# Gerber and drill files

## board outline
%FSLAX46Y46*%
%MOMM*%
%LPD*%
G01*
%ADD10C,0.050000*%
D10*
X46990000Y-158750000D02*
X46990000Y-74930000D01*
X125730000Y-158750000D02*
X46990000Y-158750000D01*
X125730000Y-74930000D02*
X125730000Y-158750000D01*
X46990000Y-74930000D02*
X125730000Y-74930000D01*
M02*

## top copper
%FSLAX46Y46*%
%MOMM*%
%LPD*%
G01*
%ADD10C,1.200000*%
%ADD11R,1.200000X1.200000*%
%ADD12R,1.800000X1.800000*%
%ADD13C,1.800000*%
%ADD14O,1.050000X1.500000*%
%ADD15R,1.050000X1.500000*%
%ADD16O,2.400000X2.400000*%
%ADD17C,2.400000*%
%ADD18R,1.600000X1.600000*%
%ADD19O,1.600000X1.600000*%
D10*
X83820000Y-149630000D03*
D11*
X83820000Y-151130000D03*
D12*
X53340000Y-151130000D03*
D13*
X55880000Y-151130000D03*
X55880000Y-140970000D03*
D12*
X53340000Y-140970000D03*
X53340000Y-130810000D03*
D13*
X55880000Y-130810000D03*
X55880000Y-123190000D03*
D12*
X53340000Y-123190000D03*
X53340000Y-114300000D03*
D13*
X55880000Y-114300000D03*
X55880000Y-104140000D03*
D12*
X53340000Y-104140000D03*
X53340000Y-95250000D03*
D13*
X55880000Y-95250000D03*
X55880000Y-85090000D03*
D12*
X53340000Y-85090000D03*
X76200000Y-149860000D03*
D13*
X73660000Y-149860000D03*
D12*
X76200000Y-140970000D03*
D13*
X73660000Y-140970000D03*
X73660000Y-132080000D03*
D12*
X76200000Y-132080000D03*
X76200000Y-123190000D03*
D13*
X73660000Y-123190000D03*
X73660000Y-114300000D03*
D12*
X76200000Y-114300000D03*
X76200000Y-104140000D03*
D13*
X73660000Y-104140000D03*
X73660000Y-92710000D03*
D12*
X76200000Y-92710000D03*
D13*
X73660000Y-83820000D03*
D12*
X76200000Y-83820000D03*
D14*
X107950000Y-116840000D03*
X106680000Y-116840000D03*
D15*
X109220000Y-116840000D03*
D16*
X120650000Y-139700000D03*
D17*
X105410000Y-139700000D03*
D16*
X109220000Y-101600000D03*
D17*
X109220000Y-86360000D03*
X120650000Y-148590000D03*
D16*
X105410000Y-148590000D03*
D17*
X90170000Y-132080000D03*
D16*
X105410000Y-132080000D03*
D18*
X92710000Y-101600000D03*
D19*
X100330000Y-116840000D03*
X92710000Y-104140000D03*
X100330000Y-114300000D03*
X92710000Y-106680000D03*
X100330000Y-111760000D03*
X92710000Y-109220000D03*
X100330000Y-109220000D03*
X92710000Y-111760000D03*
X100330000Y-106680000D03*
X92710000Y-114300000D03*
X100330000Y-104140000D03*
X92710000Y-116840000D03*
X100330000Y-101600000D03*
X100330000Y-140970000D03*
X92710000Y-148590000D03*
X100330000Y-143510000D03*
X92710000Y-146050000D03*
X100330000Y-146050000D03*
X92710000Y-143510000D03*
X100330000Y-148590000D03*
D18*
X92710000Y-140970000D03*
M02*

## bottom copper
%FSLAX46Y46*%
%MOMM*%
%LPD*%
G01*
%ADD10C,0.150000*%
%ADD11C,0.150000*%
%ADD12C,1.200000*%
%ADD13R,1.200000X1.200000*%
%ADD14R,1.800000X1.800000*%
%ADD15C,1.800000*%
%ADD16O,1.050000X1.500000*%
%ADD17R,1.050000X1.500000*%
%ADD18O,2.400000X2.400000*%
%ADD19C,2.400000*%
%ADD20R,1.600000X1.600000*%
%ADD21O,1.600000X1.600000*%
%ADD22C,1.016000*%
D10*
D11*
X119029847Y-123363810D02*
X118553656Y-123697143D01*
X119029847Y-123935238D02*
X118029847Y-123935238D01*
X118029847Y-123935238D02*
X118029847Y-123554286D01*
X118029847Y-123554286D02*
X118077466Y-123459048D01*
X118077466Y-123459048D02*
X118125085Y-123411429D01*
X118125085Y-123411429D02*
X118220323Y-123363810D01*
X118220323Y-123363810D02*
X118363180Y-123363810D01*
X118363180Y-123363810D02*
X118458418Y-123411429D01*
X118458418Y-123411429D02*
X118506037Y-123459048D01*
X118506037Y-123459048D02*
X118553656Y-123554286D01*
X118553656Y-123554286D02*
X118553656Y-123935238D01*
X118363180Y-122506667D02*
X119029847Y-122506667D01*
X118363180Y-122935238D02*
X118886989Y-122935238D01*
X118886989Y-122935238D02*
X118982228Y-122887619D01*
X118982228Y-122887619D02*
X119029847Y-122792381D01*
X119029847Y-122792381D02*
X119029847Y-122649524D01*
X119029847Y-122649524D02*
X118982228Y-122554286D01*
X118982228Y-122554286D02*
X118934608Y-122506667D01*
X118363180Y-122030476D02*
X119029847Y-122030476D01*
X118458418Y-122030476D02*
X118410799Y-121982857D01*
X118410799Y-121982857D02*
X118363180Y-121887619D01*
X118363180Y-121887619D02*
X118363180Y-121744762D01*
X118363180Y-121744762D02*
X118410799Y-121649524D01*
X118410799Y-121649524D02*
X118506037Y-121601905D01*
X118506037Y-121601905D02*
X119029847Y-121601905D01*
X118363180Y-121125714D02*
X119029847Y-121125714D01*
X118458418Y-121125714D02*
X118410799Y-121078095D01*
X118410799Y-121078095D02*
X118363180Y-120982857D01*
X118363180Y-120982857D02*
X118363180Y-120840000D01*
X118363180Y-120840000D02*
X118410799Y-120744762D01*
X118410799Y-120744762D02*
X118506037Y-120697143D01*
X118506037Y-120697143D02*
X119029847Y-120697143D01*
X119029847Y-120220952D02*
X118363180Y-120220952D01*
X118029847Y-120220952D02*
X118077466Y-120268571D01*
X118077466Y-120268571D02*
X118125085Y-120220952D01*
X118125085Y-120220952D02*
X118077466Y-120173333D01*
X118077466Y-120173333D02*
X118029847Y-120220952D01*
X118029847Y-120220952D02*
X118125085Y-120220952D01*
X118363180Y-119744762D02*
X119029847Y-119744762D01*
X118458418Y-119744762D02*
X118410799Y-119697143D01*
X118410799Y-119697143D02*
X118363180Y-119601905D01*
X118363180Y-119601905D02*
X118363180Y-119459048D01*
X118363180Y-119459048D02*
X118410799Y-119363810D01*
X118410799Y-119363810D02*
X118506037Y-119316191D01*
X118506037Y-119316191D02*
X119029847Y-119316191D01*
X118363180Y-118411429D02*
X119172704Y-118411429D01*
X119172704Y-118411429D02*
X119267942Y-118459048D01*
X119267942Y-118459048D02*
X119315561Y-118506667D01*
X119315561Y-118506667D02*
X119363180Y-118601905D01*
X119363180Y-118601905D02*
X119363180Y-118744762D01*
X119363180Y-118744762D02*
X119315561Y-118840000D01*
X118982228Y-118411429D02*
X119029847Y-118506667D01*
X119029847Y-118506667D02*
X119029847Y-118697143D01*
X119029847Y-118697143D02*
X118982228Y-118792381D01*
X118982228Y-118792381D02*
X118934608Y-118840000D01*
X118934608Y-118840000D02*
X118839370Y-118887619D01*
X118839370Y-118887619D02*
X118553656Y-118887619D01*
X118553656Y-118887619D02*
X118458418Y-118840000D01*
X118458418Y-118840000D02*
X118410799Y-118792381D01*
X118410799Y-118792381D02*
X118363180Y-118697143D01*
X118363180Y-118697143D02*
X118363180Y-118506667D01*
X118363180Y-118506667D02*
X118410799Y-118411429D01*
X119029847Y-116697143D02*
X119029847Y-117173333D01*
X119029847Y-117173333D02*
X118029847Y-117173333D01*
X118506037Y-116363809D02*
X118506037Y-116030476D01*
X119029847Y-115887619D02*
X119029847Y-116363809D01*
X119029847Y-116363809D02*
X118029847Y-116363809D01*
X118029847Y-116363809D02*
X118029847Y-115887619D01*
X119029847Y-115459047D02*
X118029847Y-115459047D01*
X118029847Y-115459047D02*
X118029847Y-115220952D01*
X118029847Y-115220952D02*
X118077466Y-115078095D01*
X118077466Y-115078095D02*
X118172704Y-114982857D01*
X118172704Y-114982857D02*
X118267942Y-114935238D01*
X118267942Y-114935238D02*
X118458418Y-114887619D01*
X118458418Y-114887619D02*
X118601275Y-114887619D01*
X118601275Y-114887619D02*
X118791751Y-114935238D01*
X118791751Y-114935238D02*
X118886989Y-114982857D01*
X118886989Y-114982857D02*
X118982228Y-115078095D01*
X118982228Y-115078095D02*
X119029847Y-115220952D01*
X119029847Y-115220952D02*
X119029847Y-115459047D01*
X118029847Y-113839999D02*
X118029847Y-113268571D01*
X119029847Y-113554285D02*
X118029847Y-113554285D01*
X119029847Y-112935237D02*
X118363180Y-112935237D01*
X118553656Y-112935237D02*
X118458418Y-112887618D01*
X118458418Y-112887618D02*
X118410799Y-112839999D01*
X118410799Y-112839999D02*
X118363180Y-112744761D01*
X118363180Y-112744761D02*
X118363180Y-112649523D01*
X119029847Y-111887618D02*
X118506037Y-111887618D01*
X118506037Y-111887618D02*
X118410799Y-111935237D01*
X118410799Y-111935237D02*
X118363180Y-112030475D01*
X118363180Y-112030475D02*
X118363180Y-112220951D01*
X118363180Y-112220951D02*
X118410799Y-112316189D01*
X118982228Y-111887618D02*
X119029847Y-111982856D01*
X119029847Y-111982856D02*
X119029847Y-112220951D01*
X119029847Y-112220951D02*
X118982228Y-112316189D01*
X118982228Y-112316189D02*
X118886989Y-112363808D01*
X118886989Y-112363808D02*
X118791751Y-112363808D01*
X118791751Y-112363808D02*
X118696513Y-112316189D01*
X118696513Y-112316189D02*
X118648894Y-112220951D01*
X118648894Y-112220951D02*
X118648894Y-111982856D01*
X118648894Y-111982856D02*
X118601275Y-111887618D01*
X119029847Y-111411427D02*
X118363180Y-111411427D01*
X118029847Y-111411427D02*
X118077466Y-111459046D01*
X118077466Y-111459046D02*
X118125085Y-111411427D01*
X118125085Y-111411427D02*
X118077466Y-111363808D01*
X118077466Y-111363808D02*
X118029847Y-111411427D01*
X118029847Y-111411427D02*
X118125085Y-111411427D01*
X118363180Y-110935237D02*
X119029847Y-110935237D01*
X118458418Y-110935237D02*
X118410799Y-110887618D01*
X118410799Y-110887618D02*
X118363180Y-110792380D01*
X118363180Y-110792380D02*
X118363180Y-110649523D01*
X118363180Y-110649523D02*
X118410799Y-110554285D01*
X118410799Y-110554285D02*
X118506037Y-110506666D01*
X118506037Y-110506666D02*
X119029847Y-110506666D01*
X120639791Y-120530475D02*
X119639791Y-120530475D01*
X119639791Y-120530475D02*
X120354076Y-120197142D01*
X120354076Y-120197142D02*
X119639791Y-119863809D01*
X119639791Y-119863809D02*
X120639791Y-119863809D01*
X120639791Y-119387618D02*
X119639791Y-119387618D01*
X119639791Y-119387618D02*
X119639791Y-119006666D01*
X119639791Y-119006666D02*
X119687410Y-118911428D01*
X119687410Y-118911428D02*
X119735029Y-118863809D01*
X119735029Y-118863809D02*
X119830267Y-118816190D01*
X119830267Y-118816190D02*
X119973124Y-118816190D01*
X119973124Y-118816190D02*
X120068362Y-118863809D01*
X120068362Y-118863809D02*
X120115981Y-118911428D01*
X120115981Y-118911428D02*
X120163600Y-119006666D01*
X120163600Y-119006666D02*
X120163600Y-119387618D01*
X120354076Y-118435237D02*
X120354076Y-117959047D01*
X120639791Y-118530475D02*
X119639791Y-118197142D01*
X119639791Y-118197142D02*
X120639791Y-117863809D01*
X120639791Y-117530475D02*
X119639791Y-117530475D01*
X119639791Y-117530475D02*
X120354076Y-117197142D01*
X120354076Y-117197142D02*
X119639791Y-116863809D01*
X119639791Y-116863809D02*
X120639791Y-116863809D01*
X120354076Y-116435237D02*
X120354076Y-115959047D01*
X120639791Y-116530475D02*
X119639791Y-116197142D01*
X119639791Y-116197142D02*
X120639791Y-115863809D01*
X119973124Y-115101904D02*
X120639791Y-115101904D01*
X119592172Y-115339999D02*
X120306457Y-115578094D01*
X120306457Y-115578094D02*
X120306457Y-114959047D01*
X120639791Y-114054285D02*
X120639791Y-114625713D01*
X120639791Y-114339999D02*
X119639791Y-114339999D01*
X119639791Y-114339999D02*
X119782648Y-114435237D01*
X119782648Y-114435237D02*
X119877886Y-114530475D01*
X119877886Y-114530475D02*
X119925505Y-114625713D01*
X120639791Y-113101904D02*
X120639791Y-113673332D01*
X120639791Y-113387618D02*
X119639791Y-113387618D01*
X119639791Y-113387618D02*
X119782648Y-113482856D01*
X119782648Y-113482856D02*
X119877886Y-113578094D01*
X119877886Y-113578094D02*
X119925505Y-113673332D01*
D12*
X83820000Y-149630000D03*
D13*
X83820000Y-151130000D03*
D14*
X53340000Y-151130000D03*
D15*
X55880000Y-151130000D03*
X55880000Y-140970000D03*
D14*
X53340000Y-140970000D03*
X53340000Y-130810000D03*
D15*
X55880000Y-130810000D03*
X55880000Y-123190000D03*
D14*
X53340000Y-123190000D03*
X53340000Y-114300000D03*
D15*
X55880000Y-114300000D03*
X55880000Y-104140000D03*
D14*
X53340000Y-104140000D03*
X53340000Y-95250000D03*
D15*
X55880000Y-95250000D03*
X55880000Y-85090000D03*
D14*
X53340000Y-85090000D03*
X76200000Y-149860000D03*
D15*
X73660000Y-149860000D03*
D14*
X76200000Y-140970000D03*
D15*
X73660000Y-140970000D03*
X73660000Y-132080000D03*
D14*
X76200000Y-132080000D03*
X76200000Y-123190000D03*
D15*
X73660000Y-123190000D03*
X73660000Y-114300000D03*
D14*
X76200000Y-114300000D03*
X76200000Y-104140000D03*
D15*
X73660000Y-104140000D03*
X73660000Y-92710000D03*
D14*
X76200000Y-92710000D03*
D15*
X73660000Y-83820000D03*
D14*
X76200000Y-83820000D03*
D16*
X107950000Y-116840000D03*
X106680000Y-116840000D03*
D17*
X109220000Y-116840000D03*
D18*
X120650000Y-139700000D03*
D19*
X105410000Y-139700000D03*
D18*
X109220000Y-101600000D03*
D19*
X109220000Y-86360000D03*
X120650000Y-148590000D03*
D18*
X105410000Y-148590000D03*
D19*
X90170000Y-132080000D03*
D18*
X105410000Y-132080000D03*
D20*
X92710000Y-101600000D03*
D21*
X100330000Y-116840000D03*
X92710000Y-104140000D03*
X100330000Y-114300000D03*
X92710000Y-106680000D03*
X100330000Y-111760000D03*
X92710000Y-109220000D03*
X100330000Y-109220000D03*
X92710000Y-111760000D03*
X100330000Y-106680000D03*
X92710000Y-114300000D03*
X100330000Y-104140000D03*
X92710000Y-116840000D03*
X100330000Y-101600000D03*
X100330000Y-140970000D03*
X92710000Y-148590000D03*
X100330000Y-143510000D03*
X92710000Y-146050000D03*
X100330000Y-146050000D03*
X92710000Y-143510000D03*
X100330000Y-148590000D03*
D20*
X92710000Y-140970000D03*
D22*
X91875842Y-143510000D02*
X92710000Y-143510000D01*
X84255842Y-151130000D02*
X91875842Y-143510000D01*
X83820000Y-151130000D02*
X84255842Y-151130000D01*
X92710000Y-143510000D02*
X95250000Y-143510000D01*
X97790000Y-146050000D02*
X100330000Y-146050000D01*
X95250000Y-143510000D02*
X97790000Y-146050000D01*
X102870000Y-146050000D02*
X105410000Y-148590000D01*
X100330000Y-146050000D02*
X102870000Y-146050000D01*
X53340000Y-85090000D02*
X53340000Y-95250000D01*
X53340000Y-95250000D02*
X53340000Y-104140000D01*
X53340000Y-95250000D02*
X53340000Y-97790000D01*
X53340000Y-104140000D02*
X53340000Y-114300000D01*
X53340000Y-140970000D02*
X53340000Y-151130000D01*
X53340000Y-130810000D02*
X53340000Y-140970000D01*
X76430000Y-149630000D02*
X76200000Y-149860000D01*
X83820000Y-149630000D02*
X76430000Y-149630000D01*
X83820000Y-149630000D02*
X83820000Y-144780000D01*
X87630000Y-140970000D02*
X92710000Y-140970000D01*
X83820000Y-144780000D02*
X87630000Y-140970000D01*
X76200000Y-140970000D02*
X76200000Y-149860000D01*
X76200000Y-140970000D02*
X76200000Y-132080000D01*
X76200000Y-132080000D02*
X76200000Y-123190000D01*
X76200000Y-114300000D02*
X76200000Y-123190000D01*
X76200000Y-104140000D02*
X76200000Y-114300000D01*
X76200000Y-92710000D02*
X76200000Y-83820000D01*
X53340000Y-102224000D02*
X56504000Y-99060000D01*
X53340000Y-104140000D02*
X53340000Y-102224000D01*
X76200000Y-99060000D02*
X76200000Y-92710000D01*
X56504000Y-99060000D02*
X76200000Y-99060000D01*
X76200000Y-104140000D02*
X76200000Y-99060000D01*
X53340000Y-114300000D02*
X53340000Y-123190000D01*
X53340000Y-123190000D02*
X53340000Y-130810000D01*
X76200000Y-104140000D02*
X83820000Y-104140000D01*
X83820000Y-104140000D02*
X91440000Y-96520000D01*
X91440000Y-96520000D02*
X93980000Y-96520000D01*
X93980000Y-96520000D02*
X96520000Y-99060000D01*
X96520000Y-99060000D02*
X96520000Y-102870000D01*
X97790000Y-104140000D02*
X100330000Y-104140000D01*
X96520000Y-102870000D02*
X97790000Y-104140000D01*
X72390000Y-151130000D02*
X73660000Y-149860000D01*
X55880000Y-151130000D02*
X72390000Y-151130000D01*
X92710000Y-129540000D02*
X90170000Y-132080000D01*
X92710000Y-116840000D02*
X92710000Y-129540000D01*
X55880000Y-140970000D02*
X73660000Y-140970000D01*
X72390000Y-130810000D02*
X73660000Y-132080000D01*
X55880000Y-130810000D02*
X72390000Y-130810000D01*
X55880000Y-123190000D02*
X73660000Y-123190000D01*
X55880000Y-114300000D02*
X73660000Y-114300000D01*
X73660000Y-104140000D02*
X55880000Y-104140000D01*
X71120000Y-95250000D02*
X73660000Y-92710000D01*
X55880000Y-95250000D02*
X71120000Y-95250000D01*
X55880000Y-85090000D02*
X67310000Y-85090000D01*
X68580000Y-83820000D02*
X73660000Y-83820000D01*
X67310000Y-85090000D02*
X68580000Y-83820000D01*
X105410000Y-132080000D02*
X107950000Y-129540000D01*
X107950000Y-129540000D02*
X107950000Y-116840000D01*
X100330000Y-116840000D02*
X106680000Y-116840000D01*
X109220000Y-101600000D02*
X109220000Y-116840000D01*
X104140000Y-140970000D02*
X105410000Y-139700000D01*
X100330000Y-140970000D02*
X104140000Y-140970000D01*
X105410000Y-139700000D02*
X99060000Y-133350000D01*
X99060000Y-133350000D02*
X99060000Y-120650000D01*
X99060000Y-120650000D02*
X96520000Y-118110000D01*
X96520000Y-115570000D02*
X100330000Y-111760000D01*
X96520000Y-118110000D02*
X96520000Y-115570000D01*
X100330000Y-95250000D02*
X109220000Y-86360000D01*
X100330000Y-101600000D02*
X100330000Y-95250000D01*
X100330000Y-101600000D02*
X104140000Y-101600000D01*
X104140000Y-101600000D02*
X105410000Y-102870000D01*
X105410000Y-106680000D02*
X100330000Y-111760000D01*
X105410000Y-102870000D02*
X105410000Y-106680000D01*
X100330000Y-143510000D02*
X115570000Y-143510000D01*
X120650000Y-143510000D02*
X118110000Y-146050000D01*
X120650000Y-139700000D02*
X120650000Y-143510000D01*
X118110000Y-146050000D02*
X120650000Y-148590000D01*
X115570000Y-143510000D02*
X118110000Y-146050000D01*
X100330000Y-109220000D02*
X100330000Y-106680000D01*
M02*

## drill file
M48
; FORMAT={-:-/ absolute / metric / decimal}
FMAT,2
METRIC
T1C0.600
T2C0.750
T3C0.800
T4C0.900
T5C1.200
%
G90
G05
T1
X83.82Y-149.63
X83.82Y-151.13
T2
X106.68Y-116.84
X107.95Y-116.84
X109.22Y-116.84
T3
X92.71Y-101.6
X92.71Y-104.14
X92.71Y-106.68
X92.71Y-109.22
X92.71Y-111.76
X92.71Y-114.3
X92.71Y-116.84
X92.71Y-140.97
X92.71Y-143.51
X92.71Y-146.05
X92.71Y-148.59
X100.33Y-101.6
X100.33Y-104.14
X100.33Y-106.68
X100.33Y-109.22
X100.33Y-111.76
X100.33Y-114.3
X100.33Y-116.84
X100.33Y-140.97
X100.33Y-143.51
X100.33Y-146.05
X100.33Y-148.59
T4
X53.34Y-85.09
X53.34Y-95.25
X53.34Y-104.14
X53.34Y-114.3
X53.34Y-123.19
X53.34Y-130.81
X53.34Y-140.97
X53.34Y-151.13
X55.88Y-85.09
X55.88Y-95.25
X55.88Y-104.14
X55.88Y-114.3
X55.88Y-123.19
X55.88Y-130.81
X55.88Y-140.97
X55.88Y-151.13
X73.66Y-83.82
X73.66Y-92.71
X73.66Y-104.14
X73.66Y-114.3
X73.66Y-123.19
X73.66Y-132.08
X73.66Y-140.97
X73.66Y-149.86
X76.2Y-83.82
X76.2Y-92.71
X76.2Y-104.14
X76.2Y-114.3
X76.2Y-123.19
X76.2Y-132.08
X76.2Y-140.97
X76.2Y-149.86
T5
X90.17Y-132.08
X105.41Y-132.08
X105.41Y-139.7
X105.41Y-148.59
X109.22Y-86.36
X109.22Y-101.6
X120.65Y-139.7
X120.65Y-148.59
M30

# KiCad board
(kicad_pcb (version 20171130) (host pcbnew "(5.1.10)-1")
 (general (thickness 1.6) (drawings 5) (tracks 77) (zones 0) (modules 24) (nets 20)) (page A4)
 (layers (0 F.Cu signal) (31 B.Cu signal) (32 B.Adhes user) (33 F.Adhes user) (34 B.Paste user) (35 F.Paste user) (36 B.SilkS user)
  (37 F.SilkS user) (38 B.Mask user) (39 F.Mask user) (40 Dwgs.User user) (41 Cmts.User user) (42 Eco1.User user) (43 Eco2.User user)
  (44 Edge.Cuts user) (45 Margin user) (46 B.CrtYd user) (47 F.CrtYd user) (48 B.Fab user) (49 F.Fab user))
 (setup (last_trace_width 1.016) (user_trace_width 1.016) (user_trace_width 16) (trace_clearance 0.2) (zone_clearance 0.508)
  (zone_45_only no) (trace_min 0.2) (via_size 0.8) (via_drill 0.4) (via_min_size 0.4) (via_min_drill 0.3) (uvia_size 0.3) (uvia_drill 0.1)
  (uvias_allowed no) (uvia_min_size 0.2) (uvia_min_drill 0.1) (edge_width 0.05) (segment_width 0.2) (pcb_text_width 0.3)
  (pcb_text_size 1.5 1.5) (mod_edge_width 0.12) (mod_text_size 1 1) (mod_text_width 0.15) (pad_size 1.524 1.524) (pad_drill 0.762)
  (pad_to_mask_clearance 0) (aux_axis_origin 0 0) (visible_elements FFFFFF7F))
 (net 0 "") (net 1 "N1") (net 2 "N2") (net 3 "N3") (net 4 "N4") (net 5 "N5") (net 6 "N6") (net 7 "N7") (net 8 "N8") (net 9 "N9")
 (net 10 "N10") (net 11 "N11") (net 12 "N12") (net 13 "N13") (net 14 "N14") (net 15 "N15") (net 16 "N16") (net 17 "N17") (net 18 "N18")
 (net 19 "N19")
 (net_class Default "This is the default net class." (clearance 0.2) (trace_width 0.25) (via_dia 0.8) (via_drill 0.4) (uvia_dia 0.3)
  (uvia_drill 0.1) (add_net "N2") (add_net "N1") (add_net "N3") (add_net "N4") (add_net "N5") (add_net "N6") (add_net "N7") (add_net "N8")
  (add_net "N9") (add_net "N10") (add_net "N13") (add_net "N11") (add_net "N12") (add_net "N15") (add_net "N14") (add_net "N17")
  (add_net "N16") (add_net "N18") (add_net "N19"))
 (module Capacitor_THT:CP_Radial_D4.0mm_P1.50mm (layer F.Cu) (at 83.82 151.13 90)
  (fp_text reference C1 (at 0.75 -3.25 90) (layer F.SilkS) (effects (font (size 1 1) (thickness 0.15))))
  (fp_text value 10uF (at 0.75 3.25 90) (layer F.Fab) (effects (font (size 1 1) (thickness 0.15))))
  (pad 2 thru_hole circle (at 1.5 0 90) (size 1.2 1.2) (drill 0.6) (layers *.Cu *.Mask) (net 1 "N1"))
  (pad 1 thru_hole rect (at 0 0 90) (size 1.2 1.2) (drill 0.6) (layers *.Cu *.Mask) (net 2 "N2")))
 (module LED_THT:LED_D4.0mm (layer F.Cu) (at 53.34 151.13)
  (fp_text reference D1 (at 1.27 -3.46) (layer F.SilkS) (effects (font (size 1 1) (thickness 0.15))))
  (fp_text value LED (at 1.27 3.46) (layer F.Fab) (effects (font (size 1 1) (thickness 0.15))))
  (pad 1 thru_hole rect (at 0 0) (size 1.8 1.8) (drill 0.9) (layers *.Cu *.Mask) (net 1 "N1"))
  (pad 2 thru_hole circle (at 2.54 0) (size 1.8 1.8) (drill 0.9) (layers *.Cu *.Mask) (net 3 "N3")))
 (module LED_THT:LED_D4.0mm (layer F.Cu) (at 53.34 140.97)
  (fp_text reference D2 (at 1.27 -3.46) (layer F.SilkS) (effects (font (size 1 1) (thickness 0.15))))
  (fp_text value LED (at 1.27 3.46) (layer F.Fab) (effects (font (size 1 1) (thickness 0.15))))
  (pad 2 thru_hole circle (at 2.54 0) (size 1.8 1.8) (drill 0.9) (layers *.Cu *.Mask) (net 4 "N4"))
  (pad 1 thru_hole rect (at 0 0) (size 1.8 1.8) (drill 0.9) (layers *.Cu *.Mask) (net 1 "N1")))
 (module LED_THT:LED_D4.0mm (layer F.Cu) (at 53.34 130.81)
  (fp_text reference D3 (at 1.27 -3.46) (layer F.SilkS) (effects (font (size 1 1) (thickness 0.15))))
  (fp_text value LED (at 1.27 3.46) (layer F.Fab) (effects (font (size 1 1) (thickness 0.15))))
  (pad 1 thru_hole rect (at 0 0) (size 1.8 1.8) (drill 0.9) (layers *.Cu *.Mask) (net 1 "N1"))
  (pad 2 thru_hole circle (at 2.54 0) (size 1.8 1.8) (drill 0.9) (layers *.Cu *.Mask) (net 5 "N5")))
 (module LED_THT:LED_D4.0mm (layer F.Cu) (at 53.34 123.19)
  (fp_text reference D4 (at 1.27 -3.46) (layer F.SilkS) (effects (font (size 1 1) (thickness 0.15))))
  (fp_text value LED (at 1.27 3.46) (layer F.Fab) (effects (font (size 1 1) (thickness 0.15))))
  (pad 2 thru_hole circle (at 2.54 0) (size 1.8 1.8) (drill 0.9) (layers *.Cu *.Mask) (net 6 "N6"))
  (pad 1 thru_hole rect (at 0 0) (size 1.8 1.8) (drill 0.9) (layers *.Cu *.Mask) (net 1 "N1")))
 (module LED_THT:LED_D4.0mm (layer F.Cu) (at 53.34 114.3)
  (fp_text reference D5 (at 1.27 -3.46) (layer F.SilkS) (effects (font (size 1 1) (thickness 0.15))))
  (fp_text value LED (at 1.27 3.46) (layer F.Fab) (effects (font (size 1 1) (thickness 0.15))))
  (pad 1 thru_hole rect (at 0 0) (size 1.8 1.8) (drill 0.9) (layers *.Cu *.Mask) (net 1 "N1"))
  (pad 2 thru_hole circle (at 2.54 0) (size 1.8 1.8) (drill 0.9) (layers *.Cu *.Mask) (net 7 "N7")))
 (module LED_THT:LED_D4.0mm (layer F.Cu) (at 53.34 104.14)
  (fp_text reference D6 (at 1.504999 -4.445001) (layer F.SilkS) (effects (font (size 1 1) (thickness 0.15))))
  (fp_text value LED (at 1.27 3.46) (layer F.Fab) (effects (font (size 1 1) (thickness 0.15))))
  (pad 2 thru_hole circle (at 2.54 0) (size 1.8 1.8) (drill 0.9) (layers *.Cu *.Mask) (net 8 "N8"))
  (pad 1 thru_hole rect (at 0 0) (size 1.8 1.8) (drill 0.9) (layers *.Cu *.Mask) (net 1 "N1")))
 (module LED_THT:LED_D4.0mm (layer F.Cu) (at 53.34 95.25)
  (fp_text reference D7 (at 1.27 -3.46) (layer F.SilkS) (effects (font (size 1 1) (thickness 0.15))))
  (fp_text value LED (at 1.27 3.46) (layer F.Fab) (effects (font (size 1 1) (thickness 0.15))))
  (pad 1 thru_hole rect (at 0 0) (size 1.8 1.8) (drill 0.9) (layers *.Cu *.Mask) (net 1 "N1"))
  (pad 2 thru_hole circle (at 2.54 0) (size 1.8 1.8) (drill 0.9) (layers *.Cu *.Mask) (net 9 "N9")))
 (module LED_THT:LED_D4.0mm (layer F.Cu) (at 53.34 85.09)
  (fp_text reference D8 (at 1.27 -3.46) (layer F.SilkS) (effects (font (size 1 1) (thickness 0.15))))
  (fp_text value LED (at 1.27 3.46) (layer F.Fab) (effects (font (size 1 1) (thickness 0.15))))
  (pad 2 thru_hole circle (at 2.54 0) (size 1.8 1.8) (drill 0.9) (layers *.Cu *.Mask) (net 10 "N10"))
  (pad 1 thru_hole rect (at 0 0) (size 1.8 1.8) (drill 0.9) (layers *.Cu *.Mask) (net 1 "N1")))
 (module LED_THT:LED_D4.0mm (layer F.Cu) (at 76.2 149.86 180)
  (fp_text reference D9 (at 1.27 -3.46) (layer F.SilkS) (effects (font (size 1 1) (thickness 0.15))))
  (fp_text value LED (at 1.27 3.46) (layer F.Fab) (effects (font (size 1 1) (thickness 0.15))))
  (pad 1 thru_hole rect (at 0 0 180) (size 1.8 1.8) (drill 0.9) (layers *.Cu *.Mask) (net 1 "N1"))
  (pad 2 thru_hole circle (at 2.54 0 180) (size 1.8 1.8) (drill 0.9) (layers *.Cu *.Mask) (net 3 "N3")))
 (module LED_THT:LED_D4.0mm (layer F.Cu) (at 76.2 140.97 180)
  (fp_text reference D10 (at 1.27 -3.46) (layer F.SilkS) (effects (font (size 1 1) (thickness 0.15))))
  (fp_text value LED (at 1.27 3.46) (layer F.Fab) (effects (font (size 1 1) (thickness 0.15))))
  (pad 1 thru_hole rect (at 0 0 180) (size 1.8 1.8) (drill 0.9) (layers *.Cu *.Mask) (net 1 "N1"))
  (pad 2 thru_hole circle (at 2.54 0 180) (size 1.8 1.8) (drill 0.9) (layers *.Cu *.Mask) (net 4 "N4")))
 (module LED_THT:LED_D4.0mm (layer F.Cu) (at 76.2 132.08 180)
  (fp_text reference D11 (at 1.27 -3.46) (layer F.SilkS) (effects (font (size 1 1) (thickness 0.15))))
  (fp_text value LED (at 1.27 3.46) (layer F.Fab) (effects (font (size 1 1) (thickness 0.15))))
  (pad 2 thru_hole circle (at 2.54 0 180) (size 1.8 1.8) (drill 0.9) (layers *.Cu *.Mask) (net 5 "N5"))
  (pad 1 thru_hole rect (at 0 0 180) (size 1.8 1.8) (drill 0.9) (layers *.Cu *.Mask) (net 1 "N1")))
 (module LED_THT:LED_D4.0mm (layer F.Cu) (at 76.2 123.19 180)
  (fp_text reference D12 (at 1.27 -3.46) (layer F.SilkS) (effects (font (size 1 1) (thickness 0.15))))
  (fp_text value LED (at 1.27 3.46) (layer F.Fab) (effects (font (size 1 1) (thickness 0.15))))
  (pad 1 thru_hole rect (at 0 0 180) (size 1.8 1.8) (drill 0.9) (layers *.Cu *.Mask) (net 1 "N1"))
  (pad 2 thru_hole circle (at 2.54 0 180) (size 1.8 1.8) (drill 0.9) (layers *.Cu *.Mask) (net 6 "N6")))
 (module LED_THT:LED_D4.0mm (layer F.Cu) (at 76.2 114.3 180)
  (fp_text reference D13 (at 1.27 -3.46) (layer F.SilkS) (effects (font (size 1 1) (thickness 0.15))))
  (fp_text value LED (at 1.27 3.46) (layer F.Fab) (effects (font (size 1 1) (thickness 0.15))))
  (pad 2 thru_hole circle (at 2.54 0 180) (size 1.8 1.8) (drill 0.9) (layers *.Cu *.Mask) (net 7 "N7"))
  (pad 1 thru_hole rect (at 0 0 180) (size 1.8 1.8) (drill 0.9) (layers *.Cu *.Mask) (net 1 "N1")))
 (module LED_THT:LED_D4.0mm (layer F.Cu) (at 76.2 104.14 180)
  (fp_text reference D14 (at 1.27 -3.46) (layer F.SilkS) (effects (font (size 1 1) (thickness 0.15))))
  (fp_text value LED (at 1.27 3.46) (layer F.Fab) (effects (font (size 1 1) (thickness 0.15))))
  (pad 1 thru_hole rect (at 0 0 180) (size 1.8 1.8) (drill 0.9) (layers *.Cu *.Mask) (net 1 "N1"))
  (pad 2 thru_hole circle (at 2.54 0 180) (size 1.8 1.8) (drill 0.9) (layers *.Cu *.Mask) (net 8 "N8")))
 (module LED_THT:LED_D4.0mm (layer F.Cu) (at 76.2 92.71 180)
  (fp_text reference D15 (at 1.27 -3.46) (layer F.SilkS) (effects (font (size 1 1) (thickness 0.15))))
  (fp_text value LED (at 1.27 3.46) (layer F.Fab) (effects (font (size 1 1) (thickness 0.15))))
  (pad 2 thru_hole circle (at 2.54 0 180) (size 1.8 1.8) (drill 0.9) (layers *.Cu *.Mask) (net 9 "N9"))
  (pad 1 thru_hole rect (at 0 0 180) (size 1.8 1.8) (drill 0.9) (layers *.Cu *.Mask) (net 1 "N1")))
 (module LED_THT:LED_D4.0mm (layer F.Cu) (at 76.2 83.82 180)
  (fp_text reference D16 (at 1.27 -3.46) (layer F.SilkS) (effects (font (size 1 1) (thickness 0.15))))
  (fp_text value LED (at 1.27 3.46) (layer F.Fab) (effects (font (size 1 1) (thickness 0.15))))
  (pad 2 thru_hole circle (at 2.54 0 180) (size 1.8 1.8) (drill 0.9) (layers *.Cu *.Mask) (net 10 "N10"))
  (pad 1 thru_hole rect (at 0 0 180) (size 1.8 1.8) (drill 0.9) (layers *.Cu *.Mask) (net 1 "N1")))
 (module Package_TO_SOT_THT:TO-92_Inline (layer F.Cu) (at 109.22 116.84 180)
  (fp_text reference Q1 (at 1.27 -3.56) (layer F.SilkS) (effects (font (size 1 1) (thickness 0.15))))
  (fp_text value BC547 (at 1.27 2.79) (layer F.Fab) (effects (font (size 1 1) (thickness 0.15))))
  (pad 2 thru_hole oval (at 1.27 0 180) (size 1.05 1.5) (drill 0.75) (layers *.Cu *.Mask) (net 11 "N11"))
  (pad 3 thru_hole oval (at 2.54 0 180) (size 1.05 1.5) (drill 0.75) (layers *.Cu *.Mask) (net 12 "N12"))
  (pad 1 thru_hole rect (at 0 0 180) (size 1.05 1.5) (drill 0.75) (layers *.Cu *.Mask) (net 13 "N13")))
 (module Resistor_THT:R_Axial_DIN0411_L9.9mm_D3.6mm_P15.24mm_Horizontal (layer F.Cu) (at 105.41 139.7)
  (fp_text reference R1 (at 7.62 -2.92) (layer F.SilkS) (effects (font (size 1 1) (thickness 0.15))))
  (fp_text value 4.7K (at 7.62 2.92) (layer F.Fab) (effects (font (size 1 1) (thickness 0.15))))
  (pad 2 thru_hole oval (at 15.24 0) (size 2.4 2.4) (drill 1.2) (layers *.Cu *.Mask) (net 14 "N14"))
  (pad 1 thru_hole circle (at 0 0) (size 2.4 2.4) (drill 1.2) (layers *.Cu *.Mask) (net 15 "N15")))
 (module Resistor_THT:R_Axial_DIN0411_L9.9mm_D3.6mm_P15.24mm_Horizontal (layer F.Cu) (at 109.22 86.36 270)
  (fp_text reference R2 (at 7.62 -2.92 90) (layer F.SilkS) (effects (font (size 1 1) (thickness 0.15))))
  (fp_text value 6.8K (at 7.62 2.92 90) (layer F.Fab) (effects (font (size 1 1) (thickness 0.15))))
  (pad 2 thru_hole oval (at 15.24 0 270) (size 2.4 2.4) (drill 1.2) (layers *.Cu *.Mask) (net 13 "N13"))
  (pad 1 thru_hole circle (at 0 0 270) (size 2.4 2.4) (drill 1.2) (layers *.Cu *.Mask) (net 15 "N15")))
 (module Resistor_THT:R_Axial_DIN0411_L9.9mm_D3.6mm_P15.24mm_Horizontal (layer F.Cu) (at 120.65 148.59 180)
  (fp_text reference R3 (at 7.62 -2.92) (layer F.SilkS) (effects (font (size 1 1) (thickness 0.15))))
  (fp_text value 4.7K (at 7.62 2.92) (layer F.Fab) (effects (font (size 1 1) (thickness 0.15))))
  (pad 1 thru_hole circle (at 0 0 180) (size 2.4 2.4) (drill 1.2) (layers *.Cu *.Mask) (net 14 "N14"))
  (pad 2 thru_hole oval (at 15.24 0 180) (size 2.4 2.4) (drill 1.2) (layers *.Cu *.Mask) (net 2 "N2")))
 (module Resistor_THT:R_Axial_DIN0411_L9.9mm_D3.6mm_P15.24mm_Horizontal (layer F.Cu) (at 90.17 132.08)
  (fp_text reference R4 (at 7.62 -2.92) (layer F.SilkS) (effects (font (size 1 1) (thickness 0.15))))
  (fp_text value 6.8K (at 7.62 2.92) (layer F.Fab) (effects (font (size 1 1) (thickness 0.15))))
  (pad 1 thru_hole circle (at 0 0) (size 2.4 2.4) (drill 1.2) (layers *.Cu *.Mask) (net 3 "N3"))
  (pad 2 thru_hole oval (at 15.24 0) (size 2.4 2.4) (drill 1.2) (layers *.Cu *.Mask) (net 11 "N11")))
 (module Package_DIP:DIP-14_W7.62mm (layer F.Cu) (at 92.71 101.6)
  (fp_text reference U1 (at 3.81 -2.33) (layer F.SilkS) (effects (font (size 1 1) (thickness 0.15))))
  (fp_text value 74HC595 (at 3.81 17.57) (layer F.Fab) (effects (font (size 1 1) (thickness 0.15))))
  (pad 1 thru_hole rect (at 0 0) (size 1.6 1.6) (drill 0.8) (layers *.Cu *.Mask) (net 9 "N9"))
  (pad 8 thru_hole oval (at 7.62 15.24) (size 1.6 1.6) (drill 0.8) (layers *.Cu *.Mask) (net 12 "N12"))
  (pad 2 thru_hole oval (at 0 2.54) (size 1.6 1.6) (drill 0.8) (layers *.Cu *.Mask) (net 8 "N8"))
  (pad 9 thru_hole oval (at 7.62 12.7) (size 1.6 1.6) (drill 0.8) (layers *.Cu *.Mask) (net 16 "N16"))
  (pad 3 thru_hole oval (at 0 5.08) (size 1.6 1.6) (drill 0.8) (layers *.Cu *.Mask) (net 7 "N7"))
  (pad 10 thru_hole oval (at 7.62 10.16) (size 1.6 1.6) (drill 0.8) (layers *.Cu *.Mask) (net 15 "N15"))
  (pad 4 thru_hole oval (at 0 7.62) (size 1.6 1.6) (drill 0.8) (layers *.Cu *.Mask) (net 6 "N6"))
  (pad 11 thru_hole oval (at 7.62 7.62) (size 1.6 1.6) (drill 0.8) (layers *.Cu *.Mask) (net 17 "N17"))
  (pad 5 thru_hole oval (at 0 10.16) (size 1.6 1.6) (drill 0.8) (layers *.Cu *.Mask) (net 5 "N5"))
  (pad 12 thru_hole oval (at 7.62 5.08) (size 1.6 1.6) (drill 0.8) (layers *.Cu *.Mask) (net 17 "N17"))
  (pad 6 thru_hole oval (at 0 12.7) (size 1.6 1.6) (drill 0.8) (layers *.Cu *.Mask) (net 4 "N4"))
  (pad 13 thru_hole oval (at 7.62 2.54) (size 1.6 1.6) (drill 0.8) (layers *.Cu *.Mask) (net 1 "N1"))
  (pad 7 thru_hole oval (at 0 15.24) (size 1.6 1.6) (drill 0.8) (layers *.Cu *.Mask) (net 3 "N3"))
  (pad 14 thru_hole oval (at 7.62 0) (size 1.6 1.6) (drill 0.8) (layers *.Cu *.Mask) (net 15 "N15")))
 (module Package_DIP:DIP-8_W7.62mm (layer F.Cu) (at 92.71 140.97)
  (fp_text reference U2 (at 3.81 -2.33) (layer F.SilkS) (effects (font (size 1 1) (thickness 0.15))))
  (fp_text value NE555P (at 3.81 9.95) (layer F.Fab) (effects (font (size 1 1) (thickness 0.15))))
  (pad 8 thru_hole oval (at 7.62 0) (size 1.6 1.6) (drill 0.8) (layers *.Cu *.Mask) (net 15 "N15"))
  (pad 4 thru_hole oval (at 0 7.62) (size 1.6 1.6) (drill 0.8) (layers *.Cu *.Mask) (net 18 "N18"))
  (pad 7 thru_hole oval (at 7.62 2.54) (size 1.6 1.6) (drill 0.8) (layers *.Cu *.Mask) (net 14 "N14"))
  (pad 3 thru_hole oval (at 0 5.08) (size 1.6 1.6) (drill 0.8) (layers *.Cu *.Mask) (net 17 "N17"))
  (pad 6 thru_hole oval (at 7.62 5.08) (size 1.6 1.6) (drill 0.8) (layers *.Cu *.Mask) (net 2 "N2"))
  (pad 2 thru_hole oval (at 0 2.54) (size 1.6 1.6) (drill 0.8) (layers *.Cu *.Mask) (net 2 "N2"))
  (pad 5 thru_hole oval (at 7.62 7.62) (size 1.6 1.6) (drill 0.8) (layers *.Cu *.Mask) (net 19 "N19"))
  (pad 1 thru_hole rect (at 0 0) (size 1.6 1.6) (drill 0.8) (layers *.Cu *.Mask) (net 1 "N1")))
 (gr_line (start 46.99 158.75) (end 46.99 74.93) (layer Edge.Cuts) (width 0.05))
 (gr_line (start 125.73 158.75) (end 46.99 158.75) (layer Edge.Cuts) (width 0.05))
 (gr_line (start 125.73 74.93) (end 125.73 158.75) (layer Edge.Cuts) (width 0.05))
 (gr_line (start 46.99 74.93) (end 125.73 74.93) (layer Edge.Cuts) (width 0.05))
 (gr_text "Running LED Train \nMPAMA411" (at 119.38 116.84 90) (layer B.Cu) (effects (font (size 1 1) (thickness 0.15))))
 (segment (start 91.875842 143.51) (end 92.71 143.51) (width 1.016) (layer B.Cu) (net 2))
 (segment (start 84.255842 151.13) (end 91.875842 143.51) (width 1.016) (layer B.Cu) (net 2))
 (segment (start 83.82 151.13) (end 84.255842 151.13) (width 1.016) (layer B.Cu) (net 2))
 (segment (start 92.71 143.51) (end 95.25 143.51) (width 1.016) (layer B.Cu) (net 2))
 (segment (start 97.79 146.05) (end 100.33 146.05) (width 1.016) (layer B.Cu) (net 2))
 (segment (start 95.25 143.51) (end 97.79 146.05) (width 1.016) (layer B.Cu) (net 2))
 (segment (start 102.87 146.05) (end 105.41 148.59) (width 1.016) (layer B.Cu) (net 2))
 (segment (start 100.33 146.05) (end 102.87 146.05) (width 1.016) (layer B.Cu) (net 2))
 (segment (start 53.34 85.09) (end 53.34 95.25) (width 1.016) (layer B.Cu) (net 1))
 (segment (start 53.34 95.25) (end 53.34 104.14) (width 1.016) (layer B.Cu) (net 1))
 (segment (start 53.34 95.25) (end 53.34 97.79) (width 1.016) (layer B.Cu) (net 1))
 (segment (start 53.34 104.14) (end 53.34 114.3) (width 1.016) (layer B.Cu) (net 1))
 (segment (start 53.34 140.97) (end 53.34 151.13) (width 1.016) (layer B.Cu) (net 1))
 (segment (start 53.34 130.81) (end 53.34 140.97) (width 1.016) (layer B.Cu) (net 1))
 (segment (start 76.43 149.63) (end 76.2 149.86) (width 1.016) (layer B.Cu) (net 1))
 (segment (start 83.82 149.63) (end 76.43 149.63) (width 1.016) (layer B.Cu) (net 1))
 (segment (start 83.82 149.63) (end 83.82 144.78) (width 1.016) (layer B.Cu) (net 1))
 (segment (start 87.63 140.97) (end 92.71 140.97) (width 1.016) (layer B.Cu) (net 1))
 (segment (start 83.82 144.78) (end 87.63 140.97) (width 1.016) (layer B.Cu) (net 1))
 (segment (start 76.2 140.97) (end 76.2 149.86) (width 1.016) (layer B.Cu) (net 1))
 (segment (start 76.2 140.97) (end 76.2 132.08) (width 1.016) (layer B.Cu) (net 1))
 (segment (start 76.2 132.08) (end 76.2 123.19) (width 1.016) (layer B.Cu) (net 1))
 (segment (start 76.2 114.3) (end 76.2 123.19) (width 1.016) (layer B.Cu) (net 1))
 (segment (start 76.2 104.14) (end 76.2 114.3) (width 1.016) (layer B.Cu) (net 1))
 (segment (start 76.2 92.71) (end 76.2 83.82) (width 1.016) (layer B.Cu) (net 1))
 (segment (start 53.34 102.224) (end 56.504 99.06) (width 1.016) (layer B.Cu) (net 1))
 (segment (start 53.34 104.14) (end 53.34 102.224) (width 1.016) (layer B.Cu) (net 1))
 (segment (start 76.2 99.06) (end 76.2 92.71) (width 1.016) (layer B.Cu) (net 1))
 (segment (start 56.504 99.06) (end 76.2 99.06) (width 1.016) (layer B.Cu) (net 1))
 (segment (start 76.2 104.14) (end 76.2 99.06) (width 1.016) (layer B.Cu) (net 1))
 (segment (start 53.34 114.3) (end 53.34 123.19) (width 1.016) (layer B.Cu) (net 1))
 (segment (start 53.34 123.19) (end 53.34 130.81) (width 1.016) (layer B.Cu) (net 1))
 (segment (start 76.2 104.14) (end 83.82 104.14) (width 1.016) (layer B.Cu) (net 1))
 (segment (start 83.82 104.14) (end 91.44 96.52) (width 1.016) (layer B.Cu) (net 1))
 (segment (start 91.44 96.52) (end 93.98 96.52) (width 1.016) (layer B.Cu) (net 1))
 (segment (start 93.98 96.52) (end 96.52 99.06) (width 1.016) (layer B.Cu) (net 1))
 (segment (start 96.52 99.06) (end 96.52 102.87) (width 1.016) (layer B.Cu) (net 1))
 (segment (start 97.79 104.14) (end 100.33 104.14) (width 1.016) (layer B.Cu) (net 1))
 (segment (start 96.52 102.87) (end 97.79 104.14) (width 1.016) (layer B.Cu) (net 1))
 (segment (start 72.39 151.13) (end 73.66 149.86) (width 1.016) (layer B.Cu) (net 3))
 (segment (start 55.88 151.13) (end 72.39 151.13) (width 1.016) (layer B.Cu) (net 3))
 (segment (start 92.71 129.54) (end 90.17 132.08) (width 1.016) (layer B.Cu) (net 3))
 (segment (start 92.71 116.84) (end 92.71 129.54) (width 1.016) (layer B.Cu) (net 3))
 (segment (start 55.88 140.97) (end 73.66 140.97) (width 1.016) (layer B.Cu) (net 4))
 (segment (start 72.39 130.81) (end 73.66 132.08) (width 1.016) (layer B.Cu) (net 5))
 (segment (start 55.88 130.81) (end 72.39 130.81) (width 1.016) (layer B.Cu) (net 5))
 (segment (start 55.88 123.19) (end 73.66 123.19) (width 1.016) (layer B.Cu) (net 6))
 (segment (start 55.88 114.3) (end 73.66 114.3) (width 1.016) (layer B.Cu) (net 7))
 (segment (start 73.66 104.14) (end 55.88 104.14) (width 1.016) (layer B.Cu) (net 8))
 (segment (start 71.12 95.25) (end 73.66 92.71) (width 1.016) (layer B.Cu) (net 9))
 (segment (start 55.88 95.25) (end 71.12 95.25) (width 1.016) (layer B.Cu) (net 9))
 (segment (start 55.88 85.09) (end 67.31 85.09) (width 1.016) (layer B.Cu) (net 10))
 (segment (start 68.58 83.82) (end 73.66 83.82) (width 1.016) (layer B.Cu) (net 10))
 (segment (start 67.31 85.09) (end 68.58 83.82) (width 1.016) (layer B.Cu) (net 10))
 (segment (start 105.41 132.08) (end 107.95 129.54) (width 1.016) (layer B.Cu) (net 11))
 (segment (start 107.95 129.54) (end 107.95 116.84) (width 1.016) (layer B.Cu) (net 11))
 (segment (start 100.33 116.84) (end 106.68 116.84) (width 1.016) (layer B.Cu) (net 12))
 (segment (start 109.22 101.6) (end 109.22 116.84) (width 1.016) (layer B.Cu) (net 13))
 (segment (start 104.14 140.97) (end 105.41 139.7) (width 1.016) (layer B.Cu) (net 15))
 (segment (start 100.33 140.97) (end 104.14 140.97) (width 1.016) (layer B.Cu) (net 15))
 (segment (start 105.41 139.7) (end 99.06 133.35) (width 1.016) (layer B.Cu) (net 15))
 (segment (start 99.06 133.35) (end 99.06 120.65) (width 1.016) (layer B.Cu) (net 15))
 (segment (start 99.06 120.65) (end 96.52 118.11) (width 1.016) (layer B.Cu) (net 15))
 (segment (start 96.52 115.57) (end 100.33 111.76) (width 1.016) (layer B.Cu) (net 15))
 (segment (start 96.52 118.11) (end 96.52 115.57) (width 1.016) (layer B.Cu) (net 15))
 (segment (start 100.33 95.25) (end 109.22 86.36) (width 1.016) (layer B.Cu) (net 15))
 (segment (start 100.33 101.6) (end 100.33 95.25) (width 1.016) (layer B.Cu) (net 15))
 (segment (start 100.33 101.6) (end 104.14 101.6) (width 1.016) (layer B.Cu) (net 15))
 (segment (start 104.14 101.6) (end 105.41 102.87) (width 1.016) (layer B.Cu) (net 15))
 (segment (start 105.41 106.68) (end 100.33 111.76) (width 1.016) (layer B.Cu) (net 15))
 (segment (start 105.41 102.87) (end 105.41 106.68) (width 1.016) (layer B.Cu) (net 15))
 (segment (start 100.33 143.51) (end 115.57 143.51) (width 1.016) (layer B.Cu) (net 14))
 (segment (start 120.65 143.51) (end 118.11 146.05) (width 1.016) (layer B.Cu) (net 14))
 (segment (start 120.65 139.7) (end 120.65 143.51) (width 1.016) (layer B.Cu) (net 14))
 (segment (start 118.11 146.05) (end 120.65 148.59) (width 1.016) (layer B.Cu) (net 14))
 (segment (start 115.57 143.51) (end 118.11 146.05) (width 1.016) (layer B.Cu) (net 14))
 (segment (start 100.33 109.22) (end 100.33 106.68) (width 1.016) (layer B.Cu) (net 17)))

